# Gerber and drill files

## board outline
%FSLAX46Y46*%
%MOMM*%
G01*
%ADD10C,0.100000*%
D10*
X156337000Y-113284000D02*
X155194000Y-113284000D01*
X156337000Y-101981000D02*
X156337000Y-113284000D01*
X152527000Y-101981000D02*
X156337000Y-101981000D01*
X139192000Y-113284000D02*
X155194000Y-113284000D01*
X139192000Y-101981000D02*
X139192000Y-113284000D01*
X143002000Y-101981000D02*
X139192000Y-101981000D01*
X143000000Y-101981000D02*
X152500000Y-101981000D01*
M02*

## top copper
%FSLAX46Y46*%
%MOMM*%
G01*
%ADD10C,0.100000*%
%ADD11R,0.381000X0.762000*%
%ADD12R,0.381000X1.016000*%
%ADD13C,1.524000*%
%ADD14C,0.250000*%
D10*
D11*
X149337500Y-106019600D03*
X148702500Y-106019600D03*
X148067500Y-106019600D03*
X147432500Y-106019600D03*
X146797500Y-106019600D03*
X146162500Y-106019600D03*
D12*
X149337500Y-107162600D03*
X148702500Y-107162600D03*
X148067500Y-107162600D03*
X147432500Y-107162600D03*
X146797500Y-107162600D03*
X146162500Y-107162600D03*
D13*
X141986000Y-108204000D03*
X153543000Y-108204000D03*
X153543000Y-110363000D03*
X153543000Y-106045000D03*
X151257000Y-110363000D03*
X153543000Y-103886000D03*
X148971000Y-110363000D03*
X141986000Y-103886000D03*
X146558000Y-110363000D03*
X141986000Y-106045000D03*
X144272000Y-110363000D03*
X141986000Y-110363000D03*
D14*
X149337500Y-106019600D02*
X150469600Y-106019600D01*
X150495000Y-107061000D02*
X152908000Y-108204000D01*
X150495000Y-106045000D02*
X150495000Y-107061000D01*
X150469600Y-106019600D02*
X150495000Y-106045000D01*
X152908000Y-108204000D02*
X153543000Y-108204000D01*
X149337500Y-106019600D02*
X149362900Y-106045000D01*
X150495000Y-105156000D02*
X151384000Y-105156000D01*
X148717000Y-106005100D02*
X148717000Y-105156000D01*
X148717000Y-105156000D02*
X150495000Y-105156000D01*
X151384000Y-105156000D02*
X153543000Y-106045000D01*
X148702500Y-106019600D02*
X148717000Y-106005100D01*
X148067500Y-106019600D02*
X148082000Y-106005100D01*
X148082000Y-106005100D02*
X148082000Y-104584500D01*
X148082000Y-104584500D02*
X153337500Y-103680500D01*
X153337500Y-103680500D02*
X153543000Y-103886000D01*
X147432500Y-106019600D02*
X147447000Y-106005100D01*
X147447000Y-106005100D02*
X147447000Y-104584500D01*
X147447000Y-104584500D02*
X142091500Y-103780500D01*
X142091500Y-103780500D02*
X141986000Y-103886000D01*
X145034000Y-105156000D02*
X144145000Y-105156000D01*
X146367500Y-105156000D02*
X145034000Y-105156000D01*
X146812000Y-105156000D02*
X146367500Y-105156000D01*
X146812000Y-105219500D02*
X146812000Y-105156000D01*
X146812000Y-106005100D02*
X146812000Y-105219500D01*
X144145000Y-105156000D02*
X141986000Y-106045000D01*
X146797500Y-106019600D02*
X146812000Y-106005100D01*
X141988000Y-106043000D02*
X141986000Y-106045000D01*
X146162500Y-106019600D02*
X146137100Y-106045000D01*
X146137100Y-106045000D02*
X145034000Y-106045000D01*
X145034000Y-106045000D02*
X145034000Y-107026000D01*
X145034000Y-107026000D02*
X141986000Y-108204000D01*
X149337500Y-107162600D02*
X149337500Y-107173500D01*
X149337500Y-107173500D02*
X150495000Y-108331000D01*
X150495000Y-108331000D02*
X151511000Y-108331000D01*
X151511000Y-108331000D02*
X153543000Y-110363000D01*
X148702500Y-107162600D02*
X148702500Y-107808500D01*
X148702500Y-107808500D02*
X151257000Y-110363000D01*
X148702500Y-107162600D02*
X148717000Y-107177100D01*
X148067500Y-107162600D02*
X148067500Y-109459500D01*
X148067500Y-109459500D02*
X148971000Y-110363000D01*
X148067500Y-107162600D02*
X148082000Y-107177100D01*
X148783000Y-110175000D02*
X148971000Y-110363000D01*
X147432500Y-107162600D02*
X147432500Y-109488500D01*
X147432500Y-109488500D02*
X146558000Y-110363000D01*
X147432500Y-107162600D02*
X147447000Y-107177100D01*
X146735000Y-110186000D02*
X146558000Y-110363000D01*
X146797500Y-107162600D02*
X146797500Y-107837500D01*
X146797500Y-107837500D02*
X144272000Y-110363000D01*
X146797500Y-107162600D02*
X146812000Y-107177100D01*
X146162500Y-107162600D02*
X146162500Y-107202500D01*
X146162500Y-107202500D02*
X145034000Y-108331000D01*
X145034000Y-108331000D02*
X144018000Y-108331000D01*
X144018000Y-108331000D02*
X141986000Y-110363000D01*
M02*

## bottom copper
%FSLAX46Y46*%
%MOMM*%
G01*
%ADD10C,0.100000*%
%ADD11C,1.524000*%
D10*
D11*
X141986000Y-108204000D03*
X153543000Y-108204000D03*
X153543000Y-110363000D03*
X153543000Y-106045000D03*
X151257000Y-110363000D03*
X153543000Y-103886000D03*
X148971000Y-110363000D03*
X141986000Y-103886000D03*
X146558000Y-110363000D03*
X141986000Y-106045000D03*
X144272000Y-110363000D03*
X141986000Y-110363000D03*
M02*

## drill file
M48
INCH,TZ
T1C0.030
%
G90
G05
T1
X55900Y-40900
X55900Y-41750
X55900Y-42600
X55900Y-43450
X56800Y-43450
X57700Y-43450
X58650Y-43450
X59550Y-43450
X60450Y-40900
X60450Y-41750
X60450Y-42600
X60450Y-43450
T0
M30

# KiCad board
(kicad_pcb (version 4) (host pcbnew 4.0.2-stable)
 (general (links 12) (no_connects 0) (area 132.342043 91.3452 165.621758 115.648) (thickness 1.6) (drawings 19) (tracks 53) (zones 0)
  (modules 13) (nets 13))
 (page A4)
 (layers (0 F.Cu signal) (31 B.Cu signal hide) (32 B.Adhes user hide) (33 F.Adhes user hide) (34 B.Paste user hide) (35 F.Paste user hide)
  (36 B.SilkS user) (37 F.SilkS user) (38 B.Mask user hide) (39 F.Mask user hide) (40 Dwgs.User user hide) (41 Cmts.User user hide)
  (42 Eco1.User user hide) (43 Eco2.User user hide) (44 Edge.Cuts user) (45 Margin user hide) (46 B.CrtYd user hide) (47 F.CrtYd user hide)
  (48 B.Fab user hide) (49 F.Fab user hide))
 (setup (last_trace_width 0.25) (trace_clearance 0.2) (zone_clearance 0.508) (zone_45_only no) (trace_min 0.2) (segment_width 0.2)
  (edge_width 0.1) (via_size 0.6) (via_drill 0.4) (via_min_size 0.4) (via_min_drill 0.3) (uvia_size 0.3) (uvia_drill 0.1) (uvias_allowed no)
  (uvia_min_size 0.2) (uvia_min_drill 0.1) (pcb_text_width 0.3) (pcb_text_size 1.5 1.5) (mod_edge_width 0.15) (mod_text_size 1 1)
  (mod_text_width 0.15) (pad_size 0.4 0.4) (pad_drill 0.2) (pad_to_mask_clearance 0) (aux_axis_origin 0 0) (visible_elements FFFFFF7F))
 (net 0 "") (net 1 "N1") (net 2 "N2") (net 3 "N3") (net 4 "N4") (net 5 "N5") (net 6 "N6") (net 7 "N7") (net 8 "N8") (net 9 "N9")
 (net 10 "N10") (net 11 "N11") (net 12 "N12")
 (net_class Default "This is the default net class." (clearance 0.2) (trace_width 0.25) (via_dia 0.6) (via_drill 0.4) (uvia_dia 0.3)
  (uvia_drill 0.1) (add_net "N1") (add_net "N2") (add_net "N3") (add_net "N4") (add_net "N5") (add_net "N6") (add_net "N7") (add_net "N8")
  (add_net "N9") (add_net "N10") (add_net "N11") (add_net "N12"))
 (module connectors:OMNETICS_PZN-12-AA (layer F.Cu) (at 147.75 105.0036)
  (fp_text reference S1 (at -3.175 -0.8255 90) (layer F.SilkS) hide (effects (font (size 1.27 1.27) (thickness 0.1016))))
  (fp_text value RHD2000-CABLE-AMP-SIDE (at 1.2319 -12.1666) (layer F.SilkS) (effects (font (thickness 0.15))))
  (pad B1 smd rect (at 1.5875 1.016 180) (size 0.381 0.762) (layers F.Cu F.Paste F.Mask) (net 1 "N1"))
  (pad B2 smd rect (at 0.9525 1.016 180) (size 0.381 0.762) (layers F.Cu F.Paste F.Mask) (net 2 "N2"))
  (pad B3 smd rect (at 0.3175 1.016 180) (size 0.381 0.762) (layers F.Cu F.Paste F.Mask) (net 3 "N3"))
  (pad B4 smd rect (at -0.3175 1.016 180) (size 0.381 0.762) (layers F.Cu F.Paste F.Mask) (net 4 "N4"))
  (pad B5 smd rect (at -0.9525 1.016 180) (size 0.381 0.762) (layers F.Cu F.Paste F.Mask) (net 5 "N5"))
  (pad B6 smd rect (at -1.5875 1.016 180) (size 0.381 0.762) (layers F.Cu F.Paste F.Mask) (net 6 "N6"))
  (pad T1 smd rect (at 1.5875 2.159 180) (size 0.381 1.016) (layers F.Cu F.Paste F.Mask) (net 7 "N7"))
  (pad T2 smd rect (at 0.9525 2.159 180) (size 0.381 1.016) (layers F.Cu F.Paste F.Mask) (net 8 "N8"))
  (pad T3 smd rect (at 0.3175 2.159 180) (size 0.381 1.016) (layers F.Cu F.Paste F.Mask) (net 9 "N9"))
  (pad T4 smd rect (at -0.3175 2.159 180) (size 0.381 1.016) (layers F.Cu F.Paste F.Mask) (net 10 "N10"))
  (pad T5 smd rect (at -0.9525 2.159 180) (size 0.381 1.016) (layers F.Cu F.Paste F.Mask) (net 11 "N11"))
  (pad T6 smd rect (at -1.5875 2.159 180) (size 0.381 1.016) (layers F.Cu F.Paste F.Mask) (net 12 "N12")))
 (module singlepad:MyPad (layer F.Cu) (at 140.716 112.014)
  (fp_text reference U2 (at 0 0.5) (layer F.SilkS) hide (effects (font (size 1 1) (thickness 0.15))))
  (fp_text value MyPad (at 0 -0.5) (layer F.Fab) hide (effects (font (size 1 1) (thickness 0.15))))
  (pad 1 thru_hole circle (at 1.27 -3.81) (size 1.524 1.524) (drill 0.762) (layers *.Cu *.Mask F.SilkS) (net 6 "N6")))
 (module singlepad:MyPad (layer F.Cu) (at 152.273 112.014)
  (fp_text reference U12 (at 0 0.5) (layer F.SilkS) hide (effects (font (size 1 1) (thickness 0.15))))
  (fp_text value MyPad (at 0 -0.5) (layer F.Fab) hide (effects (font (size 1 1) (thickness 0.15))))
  (pad 1 thru_hole circle (at 1.27 -3.81) (size 1.524 1.524) (drill 0.762) (layers *.Cu *.Mask F.SilkS) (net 1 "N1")))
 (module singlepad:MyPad (layer F.Cu) (at 152.273 114.173)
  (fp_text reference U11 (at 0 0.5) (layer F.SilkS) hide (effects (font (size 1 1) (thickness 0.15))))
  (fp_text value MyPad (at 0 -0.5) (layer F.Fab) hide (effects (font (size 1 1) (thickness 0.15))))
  (pad 1 thru_hole circle (at 1.27 -3.81) (size 1.524 1.524) (drill 0.762) (layers *.Cu *.Mask F.SilkS) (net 7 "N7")))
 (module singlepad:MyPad (layer F.Cu) (at 152.273 109.855)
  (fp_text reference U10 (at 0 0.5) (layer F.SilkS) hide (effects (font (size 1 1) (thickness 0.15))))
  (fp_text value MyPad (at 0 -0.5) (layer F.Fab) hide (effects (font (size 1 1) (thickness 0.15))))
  (pad 1 thru_hole circle (at 1.27 -3.81) (size 1.524 1.524) (drill 0.762) (layers *.Cu *.Mask F.SilkS) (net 2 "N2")))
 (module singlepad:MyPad (layer F.Cu) (at 149.987 114.173)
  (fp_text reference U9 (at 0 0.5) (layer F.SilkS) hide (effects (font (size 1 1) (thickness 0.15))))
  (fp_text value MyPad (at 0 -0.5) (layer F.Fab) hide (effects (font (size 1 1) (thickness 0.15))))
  (pad 1 thru_hole circle (at 1.27 -3.81) (size 1.524 1.524) (drill 0.762) (layers *.Cu *.Mask F.SilkS) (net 8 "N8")))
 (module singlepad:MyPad (layer F.Cu) (at 152.273 107.696)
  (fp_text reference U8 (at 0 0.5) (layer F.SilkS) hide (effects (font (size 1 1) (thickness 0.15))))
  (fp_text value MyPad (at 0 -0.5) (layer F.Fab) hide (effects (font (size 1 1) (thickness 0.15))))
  (pad 1 thru_hole circle (at 1.27 -3.81) (size 1.524 1.524) (drill 0.762) (layers *.Cu *.Mask F.SilkS) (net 3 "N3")))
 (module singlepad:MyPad (layer F.Cu) (at 147.701 114.173)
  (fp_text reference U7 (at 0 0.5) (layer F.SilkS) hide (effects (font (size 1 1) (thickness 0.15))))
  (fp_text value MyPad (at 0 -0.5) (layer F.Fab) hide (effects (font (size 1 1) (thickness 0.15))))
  (pad 1 thru_hole circle (at 1.27 -3.81) (size 1.524 1.524) (drill 0.762) (layers *.Cu *.Mask F.SilkS) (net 9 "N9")))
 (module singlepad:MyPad (layer F.Cu) (at 140.716 107.696)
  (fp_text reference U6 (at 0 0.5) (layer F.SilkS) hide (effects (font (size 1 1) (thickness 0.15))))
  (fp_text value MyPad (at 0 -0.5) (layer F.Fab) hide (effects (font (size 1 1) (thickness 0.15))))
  (pad 1 thru_hole circle (at 1.27 -3.81) (size 1.524 1.524) (drill 0.762) (layers *.Cu *.Mask F.SilkS) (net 4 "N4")))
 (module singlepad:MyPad (layer F.Cu) (at 145.288 114.173)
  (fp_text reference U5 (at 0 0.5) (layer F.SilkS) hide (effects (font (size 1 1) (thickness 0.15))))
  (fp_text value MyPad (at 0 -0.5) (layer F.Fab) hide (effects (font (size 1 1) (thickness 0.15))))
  (pad 1 thru_hole circle (at 1.27 -3.81) (size 1.524 1.524) (drill 0.762) (layers *.Cu *.Mask F.SilkS) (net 10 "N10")))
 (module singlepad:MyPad (layer F.Cu) (at 140.716 109.855)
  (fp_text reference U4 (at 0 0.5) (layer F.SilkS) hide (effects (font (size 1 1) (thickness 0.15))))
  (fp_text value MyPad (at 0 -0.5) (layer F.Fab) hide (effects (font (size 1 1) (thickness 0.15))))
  (pad 1 thru_hole circle (at 1.27 -3.81) (size 1.524 1.524) (drill 0.762) (layers *.Cu *.Mask F.SilkS) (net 5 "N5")))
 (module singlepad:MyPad (layer F.Cu) (at 143.002 114.173)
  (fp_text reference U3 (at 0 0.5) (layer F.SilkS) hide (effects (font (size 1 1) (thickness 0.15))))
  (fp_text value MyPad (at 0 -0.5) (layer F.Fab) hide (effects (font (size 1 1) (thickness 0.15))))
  (pad 1 thru_hole circle (at 1.27 -3.81) (size 1.524 1.524) (drill 0.762) (layers *.Cu *.Mask F.SilkS) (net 11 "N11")))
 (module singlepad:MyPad (layer F.Cu) (at 140.716 114.173)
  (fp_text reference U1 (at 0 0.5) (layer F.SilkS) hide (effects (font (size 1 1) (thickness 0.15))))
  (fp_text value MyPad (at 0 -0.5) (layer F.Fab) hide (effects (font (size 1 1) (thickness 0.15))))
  (pad 1 thru_hole circle (at 1.27 -3.81) (size 1.524 1.524) (drill 0.762) (layers *.Cu *.Mask F.SilkS) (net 12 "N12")))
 (gr_line (start 156.337 113.284) (end 155.194 113.284) (angle 90) (layer Edge.Cuts) (width 0.1))
 (gr_line (start 156.337 101.981) (end 156.337 113.284) (angle 90) (layer Edge.Cuts) (width 0.1))
 (gr_line (start 152.527 101.981) (end 156.337 101.981) (angle 90) (layer Edge.Cuts) (width 0.1))
 (gr_line (start 139.192 113.284) (end 155.194 113.284) (angle 90) (layer Edge.Cuts) (width 0.1))
 (gr_line (start 139.192 101.981) (end 139.192 113.284) (angle 90) (layer Edge.Cuts) (width 0.1))
 (gr_line (start 143.002 101.981) (end 139.192 101.981) (angle 90) (layer Edge.Cuts) (width 0.1))
 (gr_line (start 143 101.981) (end 152.5 101.981) (angle 90) (layer Edge.Cuts) (width 0.1))
 (segment (start 149.3375 106.0196) (end 150.4696 106.0196) (width 0.25) (layer F.Cu) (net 1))
 (segment (start 150.495 107.061) (end 152.908 108.204) (width 0.25) (layer F.Cu) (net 1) (status 20))
 (segment (start 150.495 106.045) (end 150.495 107.061) (width 0.25) (layer F.Cu) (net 1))
 (segment (start 150.4696 106.0196) (end 150.495 106.045) (width 0.25) (layer F.Cu) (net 1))
 (segment (start 152.908 108.204) (end 153.543 108.204) (width 0.25) (layer F.Cu) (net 1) (status 30))
 (segment (start 149.3375 106.0196) (end 149.3629 106.045) (width 0.25) (layer F.Cu) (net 1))
 (segment (start 150.495 105.156) (end 151.384 105.156) (width 0.25) (layer F.Cu) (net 2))
 (segment (start 148.717 106.0051) (end 148.717 105.156) (width 0.25) (layer F.Cu) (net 2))
 (segment (start 148.717 105.156) (end 150.495 105.156) (width 0.25) (layer F.Cu) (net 2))
 (segment (start 151.384 105.156) (end 153.543 106.045) (width 0.25) (layer F.Cu) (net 2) (status 20))
 (segment (start 148.7025 106.0196) (end 148.717 106.0051) (width 0.25) (layer F.Cu) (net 2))
 (segment (start 148.0675 106.0196) (end 148.082 106.0051) (width 0.25) (layer F.Cu) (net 3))
 (segment (start 148.082 106.0051) (end 148.082 104.5845) (width 0.25) (layer F.Cu) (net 3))
 (segment (start 148.082 104.5845) (end 153.3375 103.6805) (width 0.25) (layer F.Cu) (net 3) (status 20))
 (segment (start 153.3375 103.6805) (end 153.543 103.886) (width 0.25) (layer F.Cu) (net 3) (status 30))
 (segment (start 147.4325 106.0196) (end 147.447 106.0051) (width 0.25) (layer F.Cu) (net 4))
 (segment (start 147.447 106.0051) (end 147.447 104.5845) (width 0.25) (layer F.Cu) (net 4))
 (segment (start 147.447 104.5845) (end 142.0915 103.7805) (width 0.25) (layer F.Cu) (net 4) (status 20))
 (segment (start 142.0915 103.7805) (end 141.986 103.886) (width 0.25) (layer F.Cu) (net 4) (status 30))
 (segment (start 145.034 105.156) (end 144.145 105.156) (width 0.25) (layer F.Cu) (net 5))
 (segment (start 146.3675 105.156) (end 145.034 105.156) (width 0.25) (layer F.Cu) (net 5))
 (segment (start 146.812 105.156) (end 146.3675 105.156) (width 0.25) (layer F.Cu) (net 5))
 (segment (start 146.812 105.2195) (end 146.812 105.156) (width 0.25) (layer F.Cu) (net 5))
 (segment (start 146.812 106.0051) (end 146.812 105.2195) (width 0.25) (layer F.Cu) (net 5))
 (segment (start 144.145 105.156) (end 141.986 106.045) (width 0.25) (layer F.Cu) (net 5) (status 20))
 (segment (start 146.7975 106.0196) (end 146.812 106.0051) (width 0.25) (layer F.Cu) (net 5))
 (segment (start 141.988 106.043) (end 141.986 106.045) (width 0.25) (layer F.Cu) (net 5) (status 30))
 (segment (start 146.1625 106.0196) (end 146.1371 106.045) (width 0.25) (layer F.Cu) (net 6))
 (segment (start 146.1371 106.045) (end 145.034 106.045) (width 0.25) (layer F.Cu) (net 6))
 (segment (start 145.034 106.045) (end 145.034 107.026) (width 0.25) (layer F.Cu) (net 6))
 (segment (start 145.034 107.026) (end 141.986 108.204) (width 0.25) (layer F.Cu) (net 6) (status 20))
 (segment (start 149.3375 107.1626) (end 149.3375 107.1735) (width 0.25) (layer F.Cu) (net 7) (status C00000))
 (segment (start 149.3375 107.1735) (end 150.495 108.331) (width 0.25) (layer F.Cu) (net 7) (status 400000))
 (segment (start 150.495 108.331) (end 151.511 108.331) (width 0.25) (layer F.Cu) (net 7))
 (segment (start 151.511 108.331) (end 153.543 110.363) (width 0.25) (layer F.Cu) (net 7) (status 800000))
 (segment (start 148.7025 107.1626) (end 148.7025 107.8085) (width 0.25) (layer F.Cu) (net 8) (status 400000))
 (segment (start 148.7025 107.8085) (end 151.257 110.363) (width 0.25) (layer F.Cu) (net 8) (status 800000))
 (segment (start 148.7025 107.1626) (end 148.717 107.1771) (width 0.25) (layer F.Cu) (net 8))
 (segment (start 148.0675 107.1626) (end 148.0675 109.4595) (width 0.25) (layer F.Cu) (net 9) (status 400000))
 (segment (start 148.0675 109.4595) (end 148.971 110.363) (width 0.25) (layer F.Cu) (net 9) (status 800000))
 (segment (start 148.0675 107.1626) (end 148.082 107.1771) (width 0.25) (layer F.Cu) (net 9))
 (segment (start 148.783 110.175) (end 148.971 110.363) (width 0.25) (layer F.Cu) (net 9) (status 30))
 (segment (start 147.4325 107.1626) (end 147.4325 109.4885) (width 0.25) (layer F.Cu) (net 10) (status 400000))
 (segment (start 147.4325 109.4885) (end 146.558 110.363) (width 0.25) (layer F.Cu) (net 10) (status 800000))
 (segment (start 147.4325 107.1626) (end 147.447 107.1771) (width 0.25) (layer F.Cu) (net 10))
 (segment (start 146.735 110.186) (end 146.558 110.363) (width 0.25) (layer F.Cu) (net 10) (status 30))
 (segment (start 146.7975 107.1626) (end 146.7975 107.8375) (width 0.25) (layer F.Cu) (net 11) (status 400000))
 (segment (start 146.7975 107.8375) (end 144.272 110.363) (width 0.25) (layer F.Cu) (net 11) (status 800000))
 (segment (start 146.7975 107.1626) (end 146.812 107.1771) (width 0.25) (layer F.Cu) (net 11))
 (segment (start 146.1625 107.1626) (end 146.1625 107.2025) (width 0.25) (layer F.Cu) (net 12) (status C00000))
 (segment (start 146.1625 107.2025) (end 145.034 108.331) (width 0.25) (layer F.Cu) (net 12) (status 400000))
 (segment (start 145.034 108.331) (end 144.018 108.331) (width 0.25) (layer F.Cu) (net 12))
 (segment (start 144.018 108.331) (end 141.986 110.363) (width 0.25) (layer F.Cu) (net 12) (status 800000)))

